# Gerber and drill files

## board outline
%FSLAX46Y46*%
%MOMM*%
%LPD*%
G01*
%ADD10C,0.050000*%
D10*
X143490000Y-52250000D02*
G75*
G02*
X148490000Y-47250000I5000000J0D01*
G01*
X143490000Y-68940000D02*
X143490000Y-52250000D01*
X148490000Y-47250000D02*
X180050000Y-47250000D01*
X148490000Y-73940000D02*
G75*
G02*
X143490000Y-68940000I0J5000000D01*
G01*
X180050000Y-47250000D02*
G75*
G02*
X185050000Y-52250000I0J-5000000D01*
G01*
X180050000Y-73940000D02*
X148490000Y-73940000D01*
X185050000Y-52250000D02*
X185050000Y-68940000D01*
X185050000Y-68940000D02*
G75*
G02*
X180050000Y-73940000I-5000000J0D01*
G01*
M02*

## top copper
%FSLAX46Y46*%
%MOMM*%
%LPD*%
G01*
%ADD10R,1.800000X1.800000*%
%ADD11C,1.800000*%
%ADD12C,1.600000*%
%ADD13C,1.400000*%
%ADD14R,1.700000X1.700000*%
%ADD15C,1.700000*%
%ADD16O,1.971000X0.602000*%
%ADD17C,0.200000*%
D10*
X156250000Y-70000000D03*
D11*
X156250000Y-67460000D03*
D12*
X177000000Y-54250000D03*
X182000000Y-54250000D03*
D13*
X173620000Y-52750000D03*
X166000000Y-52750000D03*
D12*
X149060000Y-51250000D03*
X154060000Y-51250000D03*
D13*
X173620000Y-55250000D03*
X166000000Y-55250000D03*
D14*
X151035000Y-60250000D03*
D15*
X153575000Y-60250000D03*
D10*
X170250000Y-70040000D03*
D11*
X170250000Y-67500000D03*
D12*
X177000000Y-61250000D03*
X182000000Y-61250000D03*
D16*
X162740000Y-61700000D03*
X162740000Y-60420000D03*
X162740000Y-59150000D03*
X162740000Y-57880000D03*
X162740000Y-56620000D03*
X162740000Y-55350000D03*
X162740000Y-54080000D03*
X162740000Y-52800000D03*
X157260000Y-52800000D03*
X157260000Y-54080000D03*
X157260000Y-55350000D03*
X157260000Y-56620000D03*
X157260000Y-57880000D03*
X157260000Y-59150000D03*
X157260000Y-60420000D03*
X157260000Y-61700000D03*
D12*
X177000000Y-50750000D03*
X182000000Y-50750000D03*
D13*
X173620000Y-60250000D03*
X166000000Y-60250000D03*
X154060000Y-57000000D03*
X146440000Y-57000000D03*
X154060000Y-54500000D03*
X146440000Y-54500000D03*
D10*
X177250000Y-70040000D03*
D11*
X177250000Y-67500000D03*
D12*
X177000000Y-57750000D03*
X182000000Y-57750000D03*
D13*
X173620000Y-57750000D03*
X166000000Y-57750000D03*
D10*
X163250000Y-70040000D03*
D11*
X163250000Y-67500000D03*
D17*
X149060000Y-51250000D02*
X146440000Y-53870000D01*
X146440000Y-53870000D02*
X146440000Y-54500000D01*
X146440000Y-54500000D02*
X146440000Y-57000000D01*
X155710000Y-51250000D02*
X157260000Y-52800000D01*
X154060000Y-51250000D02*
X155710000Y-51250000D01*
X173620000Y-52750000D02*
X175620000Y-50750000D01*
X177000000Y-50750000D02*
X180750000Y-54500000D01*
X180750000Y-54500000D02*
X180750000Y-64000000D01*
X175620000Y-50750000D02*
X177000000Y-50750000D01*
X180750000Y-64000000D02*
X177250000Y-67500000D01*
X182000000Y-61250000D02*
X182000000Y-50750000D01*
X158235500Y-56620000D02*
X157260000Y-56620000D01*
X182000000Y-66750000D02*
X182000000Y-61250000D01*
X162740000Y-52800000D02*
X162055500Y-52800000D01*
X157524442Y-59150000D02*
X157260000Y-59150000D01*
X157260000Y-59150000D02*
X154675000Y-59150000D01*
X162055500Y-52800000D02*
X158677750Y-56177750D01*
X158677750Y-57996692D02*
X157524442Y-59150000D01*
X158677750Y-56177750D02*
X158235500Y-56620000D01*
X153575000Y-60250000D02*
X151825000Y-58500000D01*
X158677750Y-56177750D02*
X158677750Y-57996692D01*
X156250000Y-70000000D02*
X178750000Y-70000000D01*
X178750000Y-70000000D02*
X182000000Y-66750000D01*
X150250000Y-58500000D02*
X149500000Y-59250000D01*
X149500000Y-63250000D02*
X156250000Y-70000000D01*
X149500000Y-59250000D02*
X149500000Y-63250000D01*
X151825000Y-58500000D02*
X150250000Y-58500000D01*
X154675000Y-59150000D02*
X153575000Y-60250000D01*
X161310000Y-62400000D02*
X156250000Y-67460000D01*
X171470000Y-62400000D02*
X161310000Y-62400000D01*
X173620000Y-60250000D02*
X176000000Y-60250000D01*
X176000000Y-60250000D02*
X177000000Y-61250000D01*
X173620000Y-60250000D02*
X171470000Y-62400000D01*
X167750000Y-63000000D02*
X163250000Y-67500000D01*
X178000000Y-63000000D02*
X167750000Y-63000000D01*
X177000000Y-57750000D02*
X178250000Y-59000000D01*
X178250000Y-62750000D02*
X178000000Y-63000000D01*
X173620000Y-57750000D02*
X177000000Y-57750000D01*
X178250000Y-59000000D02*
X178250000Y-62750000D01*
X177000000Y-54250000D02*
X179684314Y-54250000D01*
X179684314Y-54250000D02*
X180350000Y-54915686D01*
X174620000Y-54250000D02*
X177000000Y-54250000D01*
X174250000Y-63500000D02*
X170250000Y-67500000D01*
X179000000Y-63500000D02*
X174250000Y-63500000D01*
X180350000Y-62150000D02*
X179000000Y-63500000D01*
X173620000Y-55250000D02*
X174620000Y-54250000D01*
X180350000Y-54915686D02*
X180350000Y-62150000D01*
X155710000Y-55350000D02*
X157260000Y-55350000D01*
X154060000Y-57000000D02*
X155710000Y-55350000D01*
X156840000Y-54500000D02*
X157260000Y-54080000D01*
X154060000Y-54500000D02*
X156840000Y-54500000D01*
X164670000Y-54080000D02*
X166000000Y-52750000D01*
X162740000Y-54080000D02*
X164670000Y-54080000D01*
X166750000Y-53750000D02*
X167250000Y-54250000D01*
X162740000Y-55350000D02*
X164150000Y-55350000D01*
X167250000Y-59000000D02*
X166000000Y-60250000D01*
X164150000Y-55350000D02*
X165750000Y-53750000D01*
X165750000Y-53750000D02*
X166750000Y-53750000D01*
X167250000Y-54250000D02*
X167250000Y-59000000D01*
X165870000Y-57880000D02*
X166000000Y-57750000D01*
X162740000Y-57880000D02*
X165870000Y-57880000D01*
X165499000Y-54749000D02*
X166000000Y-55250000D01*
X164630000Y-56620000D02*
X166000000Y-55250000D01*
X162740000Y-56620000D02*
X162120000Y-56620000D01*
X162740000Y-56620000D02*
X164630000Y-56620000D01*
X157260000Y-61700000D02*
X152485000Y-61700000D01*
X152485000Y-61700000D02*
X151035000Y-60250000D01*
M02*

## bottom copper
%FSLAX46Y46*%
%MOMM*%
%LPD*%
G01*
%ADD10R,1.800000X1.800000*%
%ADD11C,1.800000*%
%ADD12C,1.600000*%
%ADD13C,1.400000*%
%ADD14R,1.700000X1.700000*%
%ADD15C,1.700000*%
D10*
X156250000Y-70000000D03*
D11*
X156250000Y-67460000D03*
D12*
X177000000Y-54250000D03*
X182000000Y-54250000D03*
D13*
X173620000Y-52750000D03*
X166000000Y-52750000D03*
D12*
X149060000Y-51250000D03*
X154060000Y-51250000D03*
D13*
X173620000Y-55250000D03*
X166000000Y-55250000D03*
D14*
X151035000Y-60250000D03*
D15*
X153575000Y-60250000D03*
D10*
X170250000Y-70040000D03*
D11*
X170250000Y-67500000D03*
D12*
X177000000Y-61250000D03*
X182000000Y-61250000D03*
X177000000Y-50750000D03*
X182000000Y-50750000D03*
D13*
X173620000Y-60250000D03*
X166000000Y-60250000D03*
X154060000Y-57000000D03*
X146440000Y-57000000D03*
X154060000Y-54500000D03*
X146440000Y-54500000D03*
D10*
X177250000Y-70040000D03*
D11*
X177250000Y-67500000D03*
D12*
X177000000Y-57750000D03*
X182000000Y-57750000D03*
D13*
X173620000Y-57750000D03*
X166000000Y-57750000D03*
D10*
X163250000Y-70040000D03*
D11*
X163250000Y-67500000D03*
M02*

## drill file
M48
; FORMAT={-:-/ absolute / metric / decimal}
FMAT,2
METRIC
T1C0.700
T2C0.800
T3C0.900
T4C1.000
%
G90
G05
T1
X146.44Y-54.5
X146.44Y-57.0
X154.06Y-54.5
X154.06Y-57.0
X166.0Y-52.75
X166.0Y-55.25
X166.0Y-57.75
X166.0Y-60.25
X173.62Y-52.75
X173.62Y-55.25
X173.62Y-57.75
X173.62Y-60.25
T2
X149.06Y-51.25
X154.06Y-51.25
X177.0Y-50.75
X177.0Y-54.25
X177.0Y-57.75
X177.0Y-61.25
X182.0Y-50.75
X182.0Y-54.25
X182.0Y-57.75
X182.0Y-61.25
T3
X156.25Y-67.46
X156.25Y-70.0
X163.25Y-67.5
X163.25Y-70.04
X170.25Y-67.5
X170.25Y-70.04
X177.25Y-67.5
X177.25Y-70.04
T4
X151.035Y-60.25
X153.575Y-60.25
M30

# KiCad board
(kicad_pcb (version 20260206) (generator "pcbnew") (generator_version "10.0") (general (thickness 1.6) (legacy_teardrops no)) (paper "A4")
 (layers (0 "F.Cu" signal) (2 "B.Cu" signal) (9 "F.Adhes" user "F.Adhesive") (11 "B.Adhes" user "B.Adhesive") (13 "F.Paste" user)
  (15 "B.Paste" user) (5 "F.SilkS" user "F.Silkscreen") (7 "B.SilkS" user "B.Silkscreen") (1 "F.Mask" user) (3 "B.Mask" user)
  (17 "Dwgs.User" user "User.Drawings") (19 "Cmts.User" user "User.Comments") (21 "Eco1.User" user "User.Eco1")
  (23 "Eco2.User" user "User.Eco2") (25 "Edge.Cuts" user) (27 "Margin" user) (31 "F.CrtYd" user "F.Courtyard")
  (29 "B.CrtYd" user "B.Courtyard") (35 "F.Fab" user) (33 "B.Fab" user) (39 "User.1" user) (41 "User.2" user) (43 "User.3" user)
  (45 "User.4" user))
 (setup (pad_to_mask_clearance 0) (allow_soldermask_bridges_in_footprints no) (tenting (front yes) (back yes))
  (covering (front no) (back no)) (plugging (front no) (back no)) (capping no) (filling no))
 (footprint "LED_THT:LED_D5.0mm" (layer "F.Cu") (at 156.25 70 90)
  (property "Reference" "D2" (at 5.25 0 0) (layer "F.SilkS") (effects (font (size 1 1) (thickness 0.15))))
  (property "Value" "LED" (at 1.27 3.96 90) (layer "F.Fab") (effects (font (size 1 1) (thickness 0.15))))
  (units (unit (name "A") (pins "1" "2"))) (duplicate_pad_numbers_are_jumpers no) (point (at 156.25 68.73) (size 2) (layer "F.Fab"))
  (pad "1" thru_hole rect (at 0 0 90) (size 1.8 1.8) (drill 0.9) (layers "*.Cu" "*.Mask") (remove_unused_layers no) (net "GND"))
  (pad "2" thru_hole circle (at 2.54 0 90) (size 1.8 1.8) (drill 0.9) (layers "*.Cu" "*.Mask") (remove_unused_layers no) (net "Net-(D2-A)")))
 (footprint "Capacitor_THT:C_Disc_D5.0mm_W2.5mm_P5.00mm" (layer "F.Cu") (at 177 54.25)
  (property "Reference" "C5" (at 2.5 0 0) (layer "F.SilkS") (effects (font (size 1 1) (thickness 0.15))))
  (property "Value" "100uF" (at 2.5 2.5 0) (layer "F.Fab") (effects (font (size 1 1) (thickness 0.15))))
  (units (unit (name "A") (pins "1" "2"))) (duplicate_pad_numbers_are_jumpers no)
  (pad "1" thru_hole circle (at 0 0) (size 1.6 1.6) (drill 0.8) (layers "*.Cu" "*.Mask") (remove_unused_layers no) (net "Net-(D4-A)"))
  (pad "2" thru_hole circle (at 5 0) (size 1.6 1.6) (drill 0.8) (layers "*.Cu" "*.Mask") (remove_unused_layers no) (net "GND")))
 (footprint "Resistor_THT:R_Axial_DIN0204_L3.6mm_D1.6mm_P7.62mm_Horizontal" (layer "F.Cu") (at 173.62 52.75 180)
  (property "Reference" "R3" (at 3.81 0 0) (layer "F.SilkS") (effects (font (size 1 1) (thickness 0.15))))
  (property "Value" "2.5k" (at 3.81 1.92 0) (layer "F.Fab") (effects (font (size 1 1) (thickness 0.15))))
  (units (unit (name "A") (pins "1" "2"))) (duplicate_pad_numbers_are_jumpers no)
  (pad "1" thru_hole circle (at 0 0 180) (size 1.4 1.4) (drill 0.7) (layers "*.Cu" "*.Mask") (remove_unused_layers no) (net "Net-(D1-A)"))
  (pad "2" thru_hole circle (at 7.62 0 180) (size 1.4 1.4) (drill 0.7) (layers "*.Cu" "*.Mask") (remove_unused_layers no)
   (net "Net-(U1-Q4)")))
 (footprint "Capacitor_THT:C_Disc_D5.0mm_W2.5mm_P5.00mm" (layer "F.Cu") (at 149.06 51.25)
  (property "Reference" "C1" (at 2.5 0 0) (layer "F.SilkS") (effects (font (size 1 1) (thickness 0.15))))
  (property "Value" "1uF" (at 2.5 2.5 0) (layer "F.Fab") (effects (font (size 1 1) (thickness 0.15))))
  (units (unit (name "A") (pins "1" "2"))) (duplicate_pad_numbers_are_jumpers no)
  (pad "1" thru_hole circle (at 0 0) (size 1.6 1.6) (drill 0.8) (layers "*.Cu" "*.Mask") (remove_unused_layers no) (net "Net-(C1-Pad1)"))
  (pad "2" thru_hole circle (at 5 0) (size 1.6 1.6) (drill 0.8) (layers "*.Cu" "*.Mask") (remove_unused_layers no) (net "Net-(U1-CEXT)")))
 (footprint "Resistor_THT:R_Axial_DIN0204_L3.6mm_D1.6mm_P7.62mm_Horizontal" (layer "F.Cu") (at 173.62 55.25 180)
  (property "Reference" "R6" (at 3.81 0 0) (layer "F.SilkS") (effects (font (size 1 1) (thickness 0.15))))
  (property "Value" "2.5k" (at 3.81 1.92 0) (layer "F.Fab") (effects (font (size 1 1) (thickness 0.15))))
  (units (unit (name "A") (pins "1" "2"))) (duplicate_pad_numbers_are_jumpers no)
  (pad "1" thru_hole circle (at 0 0 180) (size 1.4 1.4) (drill 0.7) (layers "*.Cu" "*.Mask") (remove_unused_layers no) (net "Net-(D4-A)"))
  (pad "2" thru_hole circle (at 7.62 0 180) (size 1.4 1.4) (drill 0.7) (layers "*.Cu" "*.Mask") (remove_unused_layers no)
   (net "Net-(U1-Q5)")))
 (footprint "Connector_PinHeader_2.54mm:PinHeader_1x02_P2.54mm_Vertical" (layer "F.Cu") (at 151.035 60.25 90)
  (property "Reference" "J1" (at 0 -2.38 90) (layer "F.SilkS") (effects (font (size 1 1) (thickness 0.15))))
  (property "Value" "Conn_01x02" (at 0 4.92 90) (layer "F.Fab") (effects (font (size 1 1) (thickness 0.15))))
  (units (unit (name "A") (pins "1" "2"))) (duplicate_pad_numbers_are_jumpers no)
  (pad "1" thru_hole rect (at 0 0 90) (size 1.7 1.7) (drill 1) (layers "*.Cu" "*.Mask") (remove_unused_layers no) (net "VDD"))
  (pad "2" thru_hole circle (at 0 2.54 90) (size 1.7 1.7) (drill 1) (layers "*.Cu" "*.Mask") (remove_unused_layers no) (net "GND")))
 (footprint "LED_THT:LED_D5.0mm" (layer "F.Cu") (at 170.25 70.04 90)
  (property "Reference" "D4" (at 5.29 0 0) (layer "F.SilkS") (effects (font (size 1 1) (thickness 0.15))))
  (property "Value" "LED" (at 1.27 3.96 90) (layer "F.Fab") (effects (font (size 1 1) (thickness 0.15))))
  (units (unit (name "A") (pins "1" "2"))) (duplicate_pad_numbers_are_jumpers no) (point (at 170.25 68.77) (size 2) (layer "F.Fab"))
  (pad "1" thru_hole rect (at 0 0 90) (size 1.8 1.8) (drill 0.9) (layers "*.Cu" "*.Mask") (remove_unused_layers no) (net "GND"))
  (pad "2" thru_hole circle (at 2.54 0 90) (size 1.8 1.8) (drill 0.9) (layers "*.Cu" "*.Mask") (remove_unused_layers no) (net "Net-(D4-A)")))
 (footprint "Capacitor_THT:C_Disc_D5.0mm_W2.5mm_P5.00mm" (layer "F.Cu") (at 177 61.25)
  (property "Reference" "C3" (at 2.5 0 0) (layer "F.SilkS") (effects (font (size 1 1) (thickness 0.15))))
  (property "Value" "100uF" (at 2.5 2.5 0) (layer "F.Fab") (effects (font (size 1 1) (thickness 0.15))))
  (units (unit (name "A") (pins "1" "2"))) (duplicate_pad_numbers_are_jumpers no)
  (pad "1" thru_hole circle (at 0 0) (size 1.6 1.6) (drill 0.8) (layers "*.Cu" "*.Mask") (remove_unused_layers no) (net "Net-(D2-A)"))
  (pad "2" thru_hole circle (at 5 0) (size 1.6 1.6) (drill 0.8) (layers "*.Cu" "*.Mask") (remove_unused_layers no) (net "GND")))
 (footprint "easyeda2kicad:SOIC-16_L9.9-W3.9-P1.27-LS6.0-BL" (layer "F.Cu") (at 160 57.25 90)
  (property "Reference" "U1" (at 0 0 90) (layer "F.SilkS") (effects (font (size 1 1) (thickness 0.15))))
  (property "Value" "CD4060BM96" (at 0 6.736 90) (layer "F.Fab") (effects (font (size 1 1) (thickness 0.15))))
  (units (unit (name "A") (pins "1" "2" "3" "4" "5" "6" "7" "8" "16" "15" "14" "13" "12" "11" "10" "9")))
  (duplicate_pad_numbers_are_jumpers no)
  (pad "1" smd oval (at -4.45 2.74 90) (size 0.602 1.971) (layers "F.Cu" "F.Mask" "F.Paste") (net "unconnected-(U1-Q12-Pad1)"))
  (pad "2" smd oval (at -3.17 2.74 90) (size 0.602 1.971) (layers "F.Cu" "F.Mask" "F.Paste") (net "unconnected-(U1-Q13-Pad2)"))
  (pad "3" smd oval (at -1.9 2.74 90) (size 0.602 1.971) (layers "F.Cu" "F.Mask" "F.Paste") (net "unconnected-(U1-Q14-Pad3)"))
  (pad "4" smd oval (at -0.63 2.74 90) (size 0.602 1.971) (layers "F.Cu" "F.Mask" "F.Paste") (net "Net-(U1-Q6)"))
  (pad "5" smd oval (at 0.63 2.74 90) (size 0.602 1.971) (layers "F.Cu" "F.Mask" "F.Paste") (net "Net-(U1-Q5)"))
  (pad "6" smd oval (at 1.9 2.74 90) (size 0.602 1.971) (layers "F.Cu" "F.Mask" "F.Paste") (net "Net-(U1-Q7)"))
  (pad "7" smd oval (at 3.17 2.74 90) (size 0.602 1.971) (layers "F.Cu" "F.Mask" "F.Paste") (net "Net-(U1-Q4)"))
  (pad "8" smd oval (at 4.45 2.74 90) (size 0.602 1.971) (layers "F.Cu" "F.Mask" "F.Paste") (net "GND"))
  (pad "9" smd oval (at 4.45 -2.74 90) (size 0.602 1.971) (layers "F.Cu" "F.Mask" "F.Paste") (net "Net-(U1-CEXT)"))
  (pad "10" smd oval (at 3.17 -2.74 90) (size 0.602 1.971) (layers "F.Cu" "F.Mask" "F.Paste") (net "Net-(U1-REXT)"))
  (pad "11" smd oval (at 1.9 -2.74 90) (size 0.602 1.971) (layers "F.Cu" "F.Mask" "F.Paste") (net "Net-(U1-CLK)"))
  (pad "12" smd oval (at 0.63 -2.74 90) (size 0.602 1.971) (layers "F.Cu" "F.Mask" "F.Paste") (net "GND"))
  (pad "13" smd oval (at -0.63 -2.74 90) (size 0.602 1.971) (layers "F.Cu" "F.Mask" "F.Paste") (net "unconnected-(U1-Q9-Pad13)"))
  (pad "14" smd oval (at -1.9 -2.74 90) (size 0.602 1.971) (layers "F.Cu" "F.Mask" "F.Paste") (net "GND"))
  (pad "15" smd oval (at -3.17 -2.74 90) (size 0.602 1.971) (layers "F.Cu" "F.Mask" "F.Paste") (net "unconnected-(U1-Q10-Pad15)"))
  (pad "16" smd oval (at -4.45 -2.74 90) (size 0.602 1.971) (layers "F.Cu" "F.Mask" "F.Paste") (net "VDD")))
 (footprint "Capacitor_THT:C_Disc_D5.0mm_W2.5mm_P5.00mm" (layer "F.Cu") (at 177 50.75)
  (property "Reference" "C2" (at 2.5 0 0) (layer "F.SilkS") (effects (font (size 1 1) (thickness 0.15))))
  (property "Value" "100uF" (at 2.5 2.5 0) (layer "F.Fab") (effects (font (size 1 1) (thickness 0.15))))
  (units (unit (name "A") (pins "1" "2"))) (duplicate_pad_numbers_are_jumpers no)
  (pad "1" thru_hole circle (at 0 0) (size 1.6 1.6) (drill 0.8) (layers "*.Cu" "*.Mask") (remove_unused_layers no) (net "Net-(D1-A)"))
  (pad "2" thru_hole circle (at 5 0) (size 1.6 1.6) (drill 0.8) (layers "*.Cu" "*.Mask") (remove_unused_layers no) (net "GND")))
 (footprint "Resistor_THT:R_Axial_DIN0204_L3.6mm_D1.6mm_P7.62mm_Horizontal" (layer "F.Cu") (at 173.62 60.25 180)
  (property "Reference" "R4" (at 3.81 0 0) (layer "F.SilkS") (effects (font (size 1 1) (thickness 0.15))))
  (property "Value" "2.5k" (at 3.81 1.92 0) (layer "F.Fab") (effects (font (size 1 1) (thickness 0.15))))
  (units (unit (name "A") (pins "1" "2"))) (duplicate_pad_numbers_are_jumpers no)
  (pad "1" thru_hole circle (at 0 0 180) (size 1.4 1.4) (drill 0.7) (layers "*.Cu" "*.Mask") (remove_unused_layers no) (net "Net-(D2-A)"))
  (pad "2" thru_hole circle (at 7.62 0 180) (size 1.4 1.4) (drill 0.7) (layers "*.Cu" "*.Mask") (remove_unused_layers no)
   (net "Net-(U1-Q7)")))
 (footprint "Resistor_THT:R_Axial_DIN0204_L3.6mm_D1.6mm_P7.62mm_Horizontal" (layer "F.Cu") (at 154.06 57 180)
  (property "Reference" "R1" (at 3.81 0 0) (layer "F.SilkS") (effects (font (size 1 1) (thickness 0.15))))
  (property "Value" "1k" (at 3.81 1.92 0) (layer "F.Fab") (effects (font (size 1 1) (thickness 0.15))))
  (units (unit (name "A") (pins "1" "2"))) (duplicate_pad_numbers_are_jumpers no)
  (pad "1" thru_hole circle (at 0 0 180) (size 1.4 1.4) (drill 0.7) (layers "*.Cu" "*.Mask") (remove_unused_layers no) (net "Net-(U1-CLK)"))
  (pad "2" thru_hole circle (at 7.62 0 180) (size 1.4 1.4) (drill 0.7) (layers "*.Cu" "*.Mask") (remove_unused_layers no)
   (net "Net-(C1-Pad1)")))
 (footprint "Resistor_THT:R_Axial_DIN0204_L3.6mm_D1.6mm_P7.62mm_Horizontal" (layer "F.Cu") (at 154.06 54.5 180)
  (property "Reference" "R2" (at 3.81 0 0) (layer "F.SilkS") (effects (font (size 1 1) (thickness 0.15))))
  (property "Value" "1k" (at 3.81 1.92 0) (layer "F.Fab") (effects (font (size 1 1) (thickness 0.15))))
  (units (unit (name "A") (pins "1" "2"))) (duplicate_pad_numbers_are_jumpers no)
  (pad "1" thru_hole circle (at 0 0 180) (size 1.4 1.4) (drill 0.7) (layers "*.Cu" "*.Mask") (remove_unused_layers no) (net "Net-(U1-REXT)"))
  (pad "2" thru_hole circle (at 7.62 0 180) (size 1.4 1.4) (drill 0.7) (layers "*.Cu" "*.Mask") (remove_unused_layers no)
   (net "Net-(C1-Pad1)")))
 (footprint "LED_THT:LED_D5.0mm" (layer "F.Cu") (at 177.25 70.04 90)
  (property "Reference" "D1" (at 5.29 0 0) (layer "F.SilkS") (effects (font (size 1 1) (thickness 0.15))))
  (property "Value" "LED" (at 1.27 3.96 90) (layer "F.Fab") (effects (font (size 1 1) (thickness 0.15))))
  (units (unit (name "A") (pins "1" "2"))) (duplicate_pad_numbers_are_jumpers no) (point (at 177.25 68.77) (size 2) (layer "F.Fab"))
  (pad "1" thru_hole rect (at 0 0 90) (size 1.8 1.8) (drill 0.9) (layers "*.Cu" "*.Mask") (remove_unused_layers no) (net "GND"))
  (pad "2" thru_hole circle (at 2.54 0 90) (size 1.8 1.8) (drill 0.9) (layers "*.Cu" "*.Mask") (remove_unused_layers no) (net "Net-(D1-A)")))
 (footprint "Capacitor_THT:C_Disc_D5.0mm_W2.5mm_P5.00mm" (layer "F.Cu") (at 177 57.75)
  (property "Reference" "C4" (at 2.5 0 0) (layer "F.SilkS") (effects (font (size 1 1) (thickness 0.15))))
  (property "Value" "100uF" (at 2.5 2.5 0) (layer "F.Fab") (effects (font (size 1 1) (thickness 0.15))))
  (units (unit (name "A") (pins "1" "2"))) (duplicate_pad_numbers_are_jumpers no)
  (pad "1" thru_hole circle (at 0 0) (size 1.6 1.6) (drill 0.8) (layers "*.Cu" "*.Mask") (remove_unused_layers no) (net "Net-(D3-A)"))
  (pad "2" thru_hole circle (at 5 0) (size 1.6 1.6) (drill 0.8) (layers "*.Cu" "*.Mask") (remove_unused_layers no) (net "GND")))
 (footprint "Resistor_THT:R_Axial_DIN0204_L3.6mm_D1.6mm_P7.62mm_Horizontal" (layer "F.Cu") (at 173.62 57.75 180)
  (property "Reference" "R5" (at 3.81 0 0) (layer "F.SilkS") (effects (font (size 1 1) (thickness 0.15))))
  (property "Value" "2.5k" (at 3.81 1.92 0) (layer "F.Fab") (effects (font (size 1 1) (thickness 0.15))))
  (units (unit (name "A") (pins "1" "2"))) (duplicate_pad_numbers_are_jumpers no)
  (pad "1" thru_hole circle (at 0 0 180) (size 1.4 1.4) (drill 0.7) (layers "*.Cu" "*.Mask") (remove_unused_layers no) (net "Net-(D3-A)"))
  (pad "2" thru_hole circle (at 7.62 0 180) (size 1.4 1.4) (drill 0.7) (layers "*.Cu" "*.Mask") (remove_unused_layers no)
   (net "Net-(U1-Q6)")))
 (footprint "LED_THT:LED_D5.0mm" (layer "F.Cu") (at 163.25 70.04 90)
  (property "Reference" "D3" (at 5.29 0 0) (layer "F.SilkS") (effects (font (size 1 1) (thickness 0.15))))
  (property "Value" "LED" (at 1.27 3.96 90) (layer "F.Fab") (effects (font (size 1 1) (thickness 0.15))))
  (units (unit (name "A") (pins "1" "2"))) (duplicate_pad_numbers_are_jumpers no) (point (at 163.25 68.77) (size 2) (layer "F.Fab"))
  (pad "1" thru_hole rect (at 0 0 90) (size 1.8 1.8) (drill 0.9) (layers "*.Cu" "*.Mask") (remove_unused_layers no) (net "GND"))
  (pad "2" thru_hole circle (at 2.54 0 90) (size 1.8 1.8) (drill 0.9) (layers "*.Cu" "*.Mask") (remove_unused_layers no) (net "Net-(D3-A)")))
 (gr_arc (start 143.49 52.25) (mid 144.954466 48.714466) (end 148.49 47.25) (stroke (width 0.05) (type default)) (layer "Edge.Cuts"))
 (gr_line (start 143.49 68.94) (end 143.49 52.25) (stroke (width 0.05) (type default)) (layer "Edge.Cuts"))
 (gr_line (start 148.49 47.25) (end 180.05 47.25) (stroke (width 0.05) (type default)) (layer "Edge.Cuts"))
 (gr_arc (start 148.49 73.94) (mid 144.954466 72.475534) (end 143.49 68.94) (stroke (width 0.05) (type default)) (layer "Edge.Cuts"))
 (gr_arc (start 180.05 47.25) (mid 183.585534 48.714466) (end 185.05 52.25) (stroke (width 0.05) (type default)) (layer "Edge.Cuts"))
 (gr_line (start 180.05 73.94) (end 148.49 73.94) (stroke (width 0.05) (type default)) (layer "Edge.Cuts"))
 (gr_line (start 185.05 52.25) (end 185.05 68.94) (stroke (width 0.05) (type default)) (layer "Edge.Cuts"))
 (gr_arc (start 185.05 68.94) (mid 183.585534 72.475534) (end 180.05 73.94) (stroke (width 0.05) (type default)) (layer "Edge.Cuts"))
 (segment (start 149.06 51.25) (end 146.44 53.87) (width 0.2) (layer "F.Cu") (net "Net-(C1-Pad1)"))
 (segment (start 146.44 53.87) (end 146.44 54.5) (width 0.2) (layer "F.Cu") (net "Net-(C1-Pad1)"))
 (segment (start 146.44 54.5) (end 146.44 57) (width 0.2) (layer "F.Cu") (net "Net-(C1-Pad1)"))
 (segment (start 155.71 51.25) (end 157.26 52.8) (width 0.2) (layer "F.Cu") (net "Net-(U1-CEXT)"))
 (segment (start 154.06 51.25) (end 155.71 51.25) (width 0.2) (layer "F.Cu") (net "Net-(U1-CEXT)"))
 (segment (start 173.62 52.75) (end 175.62 50.75) (width 0.2) (layer "F.Cu") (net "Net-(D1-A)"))
 (segment (start 177 50.75) (end 180.75 54.5) (width 0.2) (layer "F.Cu") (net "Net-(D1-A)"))
 (segment (start 180.75 54.5) (end 180.75 64) (width 0.2) (layer "F.Cu") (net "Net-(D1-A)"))
 (segment (start 175.62 50.75) (end 177 50.75) (width 0.2) (layer "F.Cu") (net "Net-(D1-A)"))
 (segment (start 180.75 64) (end 177.25 67.5) (width 0.2) (layer "F.Cu") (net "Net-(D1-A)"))
 (segment (start 182 61.25) (end 182 50.75) (width 0.2) (layer "F.Cu") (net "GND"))
 (segment (start 158.2355 56.62) (end 157.26 56.62) (width 0.2) (layer "F.Cu") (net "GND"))
 (segment (start 182 66.75) (end 182 61.25) (width 0.2) (layer "F.Cu") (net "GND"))
 (segment (start 162.74 52.8) (end 162.0555 52.8) (width 0.2) (layer "F.Cu") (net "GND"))
 (segment (start 157.524442 59.15) (end 157.26 59.15) (width 0.2) (layer "F.Cu") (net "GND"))
 (segment (start 157.26 59.15) (end 154.675 59.15) (width 0.2) (layer "F.Cu") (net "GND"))
 (segment (start 162.0555 52.8) (end 158.67775 56.17775) (width 0.2) (layer "F.Cu") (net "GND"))
 (segment (start 158.67775 57.996692) (end 157.524442 59.15) (width 0.2) (layer "F.Cu") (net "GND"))
 (segment (start 158.67775 56.17775) (end 158.2355 56.62) (width 0.2) (layer "F.Cu") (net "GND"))
 (segment (start 153.575 60.25) (end 151.825 58.5) (width 0.2) (layer "F.Cu") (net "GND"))
 (segment (start 158.67775 56.17775) (end 158.67775 57.996692) (width 0.2) (layer "F.Cu") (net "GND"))
 (segment (start 156.25 70) (end 178.75 70) (width 0.2) (layer "F.Cu") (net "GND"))
 (segment (start 178.75 70) (end 182 66.75) (width 0.2) (layer "F.Cu") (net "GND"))
 (segment (start 150.25 58.5) (end 149.5 59.25) (width 0.2) (layer "F.Cu") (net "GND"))
 (segment (start 149.5 63.25) (end 156.25 70) (width 0.2) (layer "F.Cu") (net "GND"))
 (segment (start 149.5 59.25) (end 149.5 63.25) (width 0.2) (layer "F.Cu") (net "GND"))
 (segment (start 151.825 58.5) (end 150.25 58.5) (width 0.2) (layer "F.Cu") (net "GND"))
 (segment (start 154.675 59.15) (end 153.575 60.25) (width 0.2) (layer "F.Cu") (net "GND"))
 (segment (start 161.31 62.4) (end 156.25 67.46) (width 0.2) (layer "F.Cu") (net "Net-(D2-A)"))
 (segment (start 171.47 62.4) (end 161.31 62.4) (width 0.2) (layer "F.Cu") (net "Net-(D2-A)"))
 (segment (start 173.62 60.25) (end 176 60.25) (width 0.2) (layer "F.Cu") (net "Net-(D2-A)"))
 (segment (start 176 60.25) (end 177 61.25) (width 0.2) (layer "F.Cu") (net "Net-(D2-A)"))
 (segment (start 173.62 60.25) (end 171.47 62.4) (width 0.2) (layer "F.Cu") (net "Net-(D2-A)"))
 (segment (start 167.75 63) (end 163.25 67.5) (width 0.2) (layer "F.Cu") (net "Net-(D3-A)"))
 (segment (start 178 63) (end 167.75 63) (width 0.2) (layer "F.Cu") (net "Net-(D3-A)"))
 (segment (start 177 57.75) (end 178.25 59) (width 0.2) (layer "F.Cu") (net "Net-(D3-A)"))
 (segment (start 178.25 62.75) (end 178 63) (width 0.2) (layer "F.Cu") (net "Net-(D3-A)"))
 (segment (start 173.62 57.75) (end 177 57.75) (width 0.2) (layer "F.Cu") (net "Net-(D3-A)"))
 (segment (start 178.25 59) (end 178.25 62.75) (width 0.2) (layer "F.Cu") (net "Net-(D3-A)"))
 (segment (start 177 54.25) (end 179.684314 54.25) (width 0.2) (layer "F.Cu") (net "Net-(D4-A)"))
 (segment (start 179.684314 54.25) (end 180.35 54.915686) (width 0.2) (layer "F.Cu") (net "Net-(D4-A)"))
 (segment (start 174.62 54.25) (end 177 54.25) (width 0.2) (layer "F.Cu") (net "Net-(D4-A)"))
 (segment (start 174.25 63.5) (end 170.25 67.5) (width 0.2) (layer "F.Cu") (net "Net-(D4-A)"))
 (segment (start 179 63.5) (end 174.25 63.5) (width 0.2) (layer "F.Cu") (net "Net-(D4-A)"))
 (segment (start 180.35 62.15) (end 179 63.5) (width 0.2) (layer "F.Cu") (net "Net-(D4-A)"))
 (segment (start 173.62 55.25) (end 174.62 54.25) (width 0.2) (layer "F.Cu") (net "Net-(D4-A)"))
 (segment (start 180.35 54.915686) (end 180.35 62.15) (width 0.2) (layer "F.Cu") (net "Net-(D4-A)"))
 (segment (start 155.71 55.35) (end 157.26 55.35) (width 0.2) (layer "F.Cu") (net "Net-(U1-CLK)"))
 (segment (start 154.06 57) (end 155.71 55.35) (width 0.2) (layer "F.Cu") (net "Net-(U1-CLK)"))
 (segment (start 156.84 54.5) (end 157.26 54.08) (width 0.2) (layer "F.Cu") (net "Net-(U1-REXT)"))
 (segment (start 154.06 54.5) (end 156.84 54.5) (width 0.2) (layer "F.Cu") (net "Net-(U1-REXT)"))
 (segment (start 164.67 54.08) (end 166 52.75) (width 0.2) (layer "F.Cu") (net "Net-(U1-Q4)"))
 (segment (start 162.74 54.08) (end 164.67 54.08) (width 0.2) (layer "F.Cu") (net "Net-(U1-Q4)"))
 (segment (start 166.75 53.75) (end 167.25 54.25) (width 0.2) (layer "F.Cu") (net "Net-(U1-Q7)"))
 (segment (start 162.74 55.35) (end 164.15 55.35) (width 0.2) (layer "F.Cu") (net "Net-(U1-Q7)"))
 (segment (start 167.25 59) (end 166 60.25) (width 0.2) (layer "F.Cu") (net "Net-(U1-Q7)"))
 (segment (start 164.15 55.35) (end 165.75 53.75) (width 0.2) (layer "F.Cu") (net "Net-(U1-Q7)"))
 (segment (start 165.75 53.75) (end 166.75 53.75) (width 0.2) (layer "F.Cu") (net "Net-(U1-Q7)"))
 (segment (start 167.25 54.25) (end 167.25 59) (width 0.2) (layer "F.Cu") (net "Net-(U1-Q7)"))
 (segment (start 165.87 57.88) (end 166 57.75) (width 0.2) (layer "F.Cu") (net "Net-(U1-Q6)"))
 (segment (start 162.74 57.88) (end 165.87 57.88) (width 0.2) (layer "F.Cu") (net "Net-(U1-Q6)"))
 (segment (start 165.499 54.749) (end 166 55.25) (width 0.2) (layer "F.Cu") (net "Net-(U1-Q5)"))
 (segment (start 164.63 56.62) (end 166 55.25) (width 0.2) (layer "F.Cu") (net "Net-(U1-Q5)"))
 (segment (start 162.74 56.62) (end 162.12 56.62) (width 0.2) (layer "F.Cu") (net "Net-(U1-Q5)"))
 (segment (start 162.74 56.62) (end 164.63 56.62) (width 0.2) (layer "F.Cu") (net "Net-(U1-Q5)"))
 (segment (start 157.26 61.7) (end 152.485 61.7) (width 0.2) (layer "F.Cu") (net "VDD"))
 (segment (start 152.485 61.7) (end 151.035 60.25) (width 0.2) (layer "F.Cu") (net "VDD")))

